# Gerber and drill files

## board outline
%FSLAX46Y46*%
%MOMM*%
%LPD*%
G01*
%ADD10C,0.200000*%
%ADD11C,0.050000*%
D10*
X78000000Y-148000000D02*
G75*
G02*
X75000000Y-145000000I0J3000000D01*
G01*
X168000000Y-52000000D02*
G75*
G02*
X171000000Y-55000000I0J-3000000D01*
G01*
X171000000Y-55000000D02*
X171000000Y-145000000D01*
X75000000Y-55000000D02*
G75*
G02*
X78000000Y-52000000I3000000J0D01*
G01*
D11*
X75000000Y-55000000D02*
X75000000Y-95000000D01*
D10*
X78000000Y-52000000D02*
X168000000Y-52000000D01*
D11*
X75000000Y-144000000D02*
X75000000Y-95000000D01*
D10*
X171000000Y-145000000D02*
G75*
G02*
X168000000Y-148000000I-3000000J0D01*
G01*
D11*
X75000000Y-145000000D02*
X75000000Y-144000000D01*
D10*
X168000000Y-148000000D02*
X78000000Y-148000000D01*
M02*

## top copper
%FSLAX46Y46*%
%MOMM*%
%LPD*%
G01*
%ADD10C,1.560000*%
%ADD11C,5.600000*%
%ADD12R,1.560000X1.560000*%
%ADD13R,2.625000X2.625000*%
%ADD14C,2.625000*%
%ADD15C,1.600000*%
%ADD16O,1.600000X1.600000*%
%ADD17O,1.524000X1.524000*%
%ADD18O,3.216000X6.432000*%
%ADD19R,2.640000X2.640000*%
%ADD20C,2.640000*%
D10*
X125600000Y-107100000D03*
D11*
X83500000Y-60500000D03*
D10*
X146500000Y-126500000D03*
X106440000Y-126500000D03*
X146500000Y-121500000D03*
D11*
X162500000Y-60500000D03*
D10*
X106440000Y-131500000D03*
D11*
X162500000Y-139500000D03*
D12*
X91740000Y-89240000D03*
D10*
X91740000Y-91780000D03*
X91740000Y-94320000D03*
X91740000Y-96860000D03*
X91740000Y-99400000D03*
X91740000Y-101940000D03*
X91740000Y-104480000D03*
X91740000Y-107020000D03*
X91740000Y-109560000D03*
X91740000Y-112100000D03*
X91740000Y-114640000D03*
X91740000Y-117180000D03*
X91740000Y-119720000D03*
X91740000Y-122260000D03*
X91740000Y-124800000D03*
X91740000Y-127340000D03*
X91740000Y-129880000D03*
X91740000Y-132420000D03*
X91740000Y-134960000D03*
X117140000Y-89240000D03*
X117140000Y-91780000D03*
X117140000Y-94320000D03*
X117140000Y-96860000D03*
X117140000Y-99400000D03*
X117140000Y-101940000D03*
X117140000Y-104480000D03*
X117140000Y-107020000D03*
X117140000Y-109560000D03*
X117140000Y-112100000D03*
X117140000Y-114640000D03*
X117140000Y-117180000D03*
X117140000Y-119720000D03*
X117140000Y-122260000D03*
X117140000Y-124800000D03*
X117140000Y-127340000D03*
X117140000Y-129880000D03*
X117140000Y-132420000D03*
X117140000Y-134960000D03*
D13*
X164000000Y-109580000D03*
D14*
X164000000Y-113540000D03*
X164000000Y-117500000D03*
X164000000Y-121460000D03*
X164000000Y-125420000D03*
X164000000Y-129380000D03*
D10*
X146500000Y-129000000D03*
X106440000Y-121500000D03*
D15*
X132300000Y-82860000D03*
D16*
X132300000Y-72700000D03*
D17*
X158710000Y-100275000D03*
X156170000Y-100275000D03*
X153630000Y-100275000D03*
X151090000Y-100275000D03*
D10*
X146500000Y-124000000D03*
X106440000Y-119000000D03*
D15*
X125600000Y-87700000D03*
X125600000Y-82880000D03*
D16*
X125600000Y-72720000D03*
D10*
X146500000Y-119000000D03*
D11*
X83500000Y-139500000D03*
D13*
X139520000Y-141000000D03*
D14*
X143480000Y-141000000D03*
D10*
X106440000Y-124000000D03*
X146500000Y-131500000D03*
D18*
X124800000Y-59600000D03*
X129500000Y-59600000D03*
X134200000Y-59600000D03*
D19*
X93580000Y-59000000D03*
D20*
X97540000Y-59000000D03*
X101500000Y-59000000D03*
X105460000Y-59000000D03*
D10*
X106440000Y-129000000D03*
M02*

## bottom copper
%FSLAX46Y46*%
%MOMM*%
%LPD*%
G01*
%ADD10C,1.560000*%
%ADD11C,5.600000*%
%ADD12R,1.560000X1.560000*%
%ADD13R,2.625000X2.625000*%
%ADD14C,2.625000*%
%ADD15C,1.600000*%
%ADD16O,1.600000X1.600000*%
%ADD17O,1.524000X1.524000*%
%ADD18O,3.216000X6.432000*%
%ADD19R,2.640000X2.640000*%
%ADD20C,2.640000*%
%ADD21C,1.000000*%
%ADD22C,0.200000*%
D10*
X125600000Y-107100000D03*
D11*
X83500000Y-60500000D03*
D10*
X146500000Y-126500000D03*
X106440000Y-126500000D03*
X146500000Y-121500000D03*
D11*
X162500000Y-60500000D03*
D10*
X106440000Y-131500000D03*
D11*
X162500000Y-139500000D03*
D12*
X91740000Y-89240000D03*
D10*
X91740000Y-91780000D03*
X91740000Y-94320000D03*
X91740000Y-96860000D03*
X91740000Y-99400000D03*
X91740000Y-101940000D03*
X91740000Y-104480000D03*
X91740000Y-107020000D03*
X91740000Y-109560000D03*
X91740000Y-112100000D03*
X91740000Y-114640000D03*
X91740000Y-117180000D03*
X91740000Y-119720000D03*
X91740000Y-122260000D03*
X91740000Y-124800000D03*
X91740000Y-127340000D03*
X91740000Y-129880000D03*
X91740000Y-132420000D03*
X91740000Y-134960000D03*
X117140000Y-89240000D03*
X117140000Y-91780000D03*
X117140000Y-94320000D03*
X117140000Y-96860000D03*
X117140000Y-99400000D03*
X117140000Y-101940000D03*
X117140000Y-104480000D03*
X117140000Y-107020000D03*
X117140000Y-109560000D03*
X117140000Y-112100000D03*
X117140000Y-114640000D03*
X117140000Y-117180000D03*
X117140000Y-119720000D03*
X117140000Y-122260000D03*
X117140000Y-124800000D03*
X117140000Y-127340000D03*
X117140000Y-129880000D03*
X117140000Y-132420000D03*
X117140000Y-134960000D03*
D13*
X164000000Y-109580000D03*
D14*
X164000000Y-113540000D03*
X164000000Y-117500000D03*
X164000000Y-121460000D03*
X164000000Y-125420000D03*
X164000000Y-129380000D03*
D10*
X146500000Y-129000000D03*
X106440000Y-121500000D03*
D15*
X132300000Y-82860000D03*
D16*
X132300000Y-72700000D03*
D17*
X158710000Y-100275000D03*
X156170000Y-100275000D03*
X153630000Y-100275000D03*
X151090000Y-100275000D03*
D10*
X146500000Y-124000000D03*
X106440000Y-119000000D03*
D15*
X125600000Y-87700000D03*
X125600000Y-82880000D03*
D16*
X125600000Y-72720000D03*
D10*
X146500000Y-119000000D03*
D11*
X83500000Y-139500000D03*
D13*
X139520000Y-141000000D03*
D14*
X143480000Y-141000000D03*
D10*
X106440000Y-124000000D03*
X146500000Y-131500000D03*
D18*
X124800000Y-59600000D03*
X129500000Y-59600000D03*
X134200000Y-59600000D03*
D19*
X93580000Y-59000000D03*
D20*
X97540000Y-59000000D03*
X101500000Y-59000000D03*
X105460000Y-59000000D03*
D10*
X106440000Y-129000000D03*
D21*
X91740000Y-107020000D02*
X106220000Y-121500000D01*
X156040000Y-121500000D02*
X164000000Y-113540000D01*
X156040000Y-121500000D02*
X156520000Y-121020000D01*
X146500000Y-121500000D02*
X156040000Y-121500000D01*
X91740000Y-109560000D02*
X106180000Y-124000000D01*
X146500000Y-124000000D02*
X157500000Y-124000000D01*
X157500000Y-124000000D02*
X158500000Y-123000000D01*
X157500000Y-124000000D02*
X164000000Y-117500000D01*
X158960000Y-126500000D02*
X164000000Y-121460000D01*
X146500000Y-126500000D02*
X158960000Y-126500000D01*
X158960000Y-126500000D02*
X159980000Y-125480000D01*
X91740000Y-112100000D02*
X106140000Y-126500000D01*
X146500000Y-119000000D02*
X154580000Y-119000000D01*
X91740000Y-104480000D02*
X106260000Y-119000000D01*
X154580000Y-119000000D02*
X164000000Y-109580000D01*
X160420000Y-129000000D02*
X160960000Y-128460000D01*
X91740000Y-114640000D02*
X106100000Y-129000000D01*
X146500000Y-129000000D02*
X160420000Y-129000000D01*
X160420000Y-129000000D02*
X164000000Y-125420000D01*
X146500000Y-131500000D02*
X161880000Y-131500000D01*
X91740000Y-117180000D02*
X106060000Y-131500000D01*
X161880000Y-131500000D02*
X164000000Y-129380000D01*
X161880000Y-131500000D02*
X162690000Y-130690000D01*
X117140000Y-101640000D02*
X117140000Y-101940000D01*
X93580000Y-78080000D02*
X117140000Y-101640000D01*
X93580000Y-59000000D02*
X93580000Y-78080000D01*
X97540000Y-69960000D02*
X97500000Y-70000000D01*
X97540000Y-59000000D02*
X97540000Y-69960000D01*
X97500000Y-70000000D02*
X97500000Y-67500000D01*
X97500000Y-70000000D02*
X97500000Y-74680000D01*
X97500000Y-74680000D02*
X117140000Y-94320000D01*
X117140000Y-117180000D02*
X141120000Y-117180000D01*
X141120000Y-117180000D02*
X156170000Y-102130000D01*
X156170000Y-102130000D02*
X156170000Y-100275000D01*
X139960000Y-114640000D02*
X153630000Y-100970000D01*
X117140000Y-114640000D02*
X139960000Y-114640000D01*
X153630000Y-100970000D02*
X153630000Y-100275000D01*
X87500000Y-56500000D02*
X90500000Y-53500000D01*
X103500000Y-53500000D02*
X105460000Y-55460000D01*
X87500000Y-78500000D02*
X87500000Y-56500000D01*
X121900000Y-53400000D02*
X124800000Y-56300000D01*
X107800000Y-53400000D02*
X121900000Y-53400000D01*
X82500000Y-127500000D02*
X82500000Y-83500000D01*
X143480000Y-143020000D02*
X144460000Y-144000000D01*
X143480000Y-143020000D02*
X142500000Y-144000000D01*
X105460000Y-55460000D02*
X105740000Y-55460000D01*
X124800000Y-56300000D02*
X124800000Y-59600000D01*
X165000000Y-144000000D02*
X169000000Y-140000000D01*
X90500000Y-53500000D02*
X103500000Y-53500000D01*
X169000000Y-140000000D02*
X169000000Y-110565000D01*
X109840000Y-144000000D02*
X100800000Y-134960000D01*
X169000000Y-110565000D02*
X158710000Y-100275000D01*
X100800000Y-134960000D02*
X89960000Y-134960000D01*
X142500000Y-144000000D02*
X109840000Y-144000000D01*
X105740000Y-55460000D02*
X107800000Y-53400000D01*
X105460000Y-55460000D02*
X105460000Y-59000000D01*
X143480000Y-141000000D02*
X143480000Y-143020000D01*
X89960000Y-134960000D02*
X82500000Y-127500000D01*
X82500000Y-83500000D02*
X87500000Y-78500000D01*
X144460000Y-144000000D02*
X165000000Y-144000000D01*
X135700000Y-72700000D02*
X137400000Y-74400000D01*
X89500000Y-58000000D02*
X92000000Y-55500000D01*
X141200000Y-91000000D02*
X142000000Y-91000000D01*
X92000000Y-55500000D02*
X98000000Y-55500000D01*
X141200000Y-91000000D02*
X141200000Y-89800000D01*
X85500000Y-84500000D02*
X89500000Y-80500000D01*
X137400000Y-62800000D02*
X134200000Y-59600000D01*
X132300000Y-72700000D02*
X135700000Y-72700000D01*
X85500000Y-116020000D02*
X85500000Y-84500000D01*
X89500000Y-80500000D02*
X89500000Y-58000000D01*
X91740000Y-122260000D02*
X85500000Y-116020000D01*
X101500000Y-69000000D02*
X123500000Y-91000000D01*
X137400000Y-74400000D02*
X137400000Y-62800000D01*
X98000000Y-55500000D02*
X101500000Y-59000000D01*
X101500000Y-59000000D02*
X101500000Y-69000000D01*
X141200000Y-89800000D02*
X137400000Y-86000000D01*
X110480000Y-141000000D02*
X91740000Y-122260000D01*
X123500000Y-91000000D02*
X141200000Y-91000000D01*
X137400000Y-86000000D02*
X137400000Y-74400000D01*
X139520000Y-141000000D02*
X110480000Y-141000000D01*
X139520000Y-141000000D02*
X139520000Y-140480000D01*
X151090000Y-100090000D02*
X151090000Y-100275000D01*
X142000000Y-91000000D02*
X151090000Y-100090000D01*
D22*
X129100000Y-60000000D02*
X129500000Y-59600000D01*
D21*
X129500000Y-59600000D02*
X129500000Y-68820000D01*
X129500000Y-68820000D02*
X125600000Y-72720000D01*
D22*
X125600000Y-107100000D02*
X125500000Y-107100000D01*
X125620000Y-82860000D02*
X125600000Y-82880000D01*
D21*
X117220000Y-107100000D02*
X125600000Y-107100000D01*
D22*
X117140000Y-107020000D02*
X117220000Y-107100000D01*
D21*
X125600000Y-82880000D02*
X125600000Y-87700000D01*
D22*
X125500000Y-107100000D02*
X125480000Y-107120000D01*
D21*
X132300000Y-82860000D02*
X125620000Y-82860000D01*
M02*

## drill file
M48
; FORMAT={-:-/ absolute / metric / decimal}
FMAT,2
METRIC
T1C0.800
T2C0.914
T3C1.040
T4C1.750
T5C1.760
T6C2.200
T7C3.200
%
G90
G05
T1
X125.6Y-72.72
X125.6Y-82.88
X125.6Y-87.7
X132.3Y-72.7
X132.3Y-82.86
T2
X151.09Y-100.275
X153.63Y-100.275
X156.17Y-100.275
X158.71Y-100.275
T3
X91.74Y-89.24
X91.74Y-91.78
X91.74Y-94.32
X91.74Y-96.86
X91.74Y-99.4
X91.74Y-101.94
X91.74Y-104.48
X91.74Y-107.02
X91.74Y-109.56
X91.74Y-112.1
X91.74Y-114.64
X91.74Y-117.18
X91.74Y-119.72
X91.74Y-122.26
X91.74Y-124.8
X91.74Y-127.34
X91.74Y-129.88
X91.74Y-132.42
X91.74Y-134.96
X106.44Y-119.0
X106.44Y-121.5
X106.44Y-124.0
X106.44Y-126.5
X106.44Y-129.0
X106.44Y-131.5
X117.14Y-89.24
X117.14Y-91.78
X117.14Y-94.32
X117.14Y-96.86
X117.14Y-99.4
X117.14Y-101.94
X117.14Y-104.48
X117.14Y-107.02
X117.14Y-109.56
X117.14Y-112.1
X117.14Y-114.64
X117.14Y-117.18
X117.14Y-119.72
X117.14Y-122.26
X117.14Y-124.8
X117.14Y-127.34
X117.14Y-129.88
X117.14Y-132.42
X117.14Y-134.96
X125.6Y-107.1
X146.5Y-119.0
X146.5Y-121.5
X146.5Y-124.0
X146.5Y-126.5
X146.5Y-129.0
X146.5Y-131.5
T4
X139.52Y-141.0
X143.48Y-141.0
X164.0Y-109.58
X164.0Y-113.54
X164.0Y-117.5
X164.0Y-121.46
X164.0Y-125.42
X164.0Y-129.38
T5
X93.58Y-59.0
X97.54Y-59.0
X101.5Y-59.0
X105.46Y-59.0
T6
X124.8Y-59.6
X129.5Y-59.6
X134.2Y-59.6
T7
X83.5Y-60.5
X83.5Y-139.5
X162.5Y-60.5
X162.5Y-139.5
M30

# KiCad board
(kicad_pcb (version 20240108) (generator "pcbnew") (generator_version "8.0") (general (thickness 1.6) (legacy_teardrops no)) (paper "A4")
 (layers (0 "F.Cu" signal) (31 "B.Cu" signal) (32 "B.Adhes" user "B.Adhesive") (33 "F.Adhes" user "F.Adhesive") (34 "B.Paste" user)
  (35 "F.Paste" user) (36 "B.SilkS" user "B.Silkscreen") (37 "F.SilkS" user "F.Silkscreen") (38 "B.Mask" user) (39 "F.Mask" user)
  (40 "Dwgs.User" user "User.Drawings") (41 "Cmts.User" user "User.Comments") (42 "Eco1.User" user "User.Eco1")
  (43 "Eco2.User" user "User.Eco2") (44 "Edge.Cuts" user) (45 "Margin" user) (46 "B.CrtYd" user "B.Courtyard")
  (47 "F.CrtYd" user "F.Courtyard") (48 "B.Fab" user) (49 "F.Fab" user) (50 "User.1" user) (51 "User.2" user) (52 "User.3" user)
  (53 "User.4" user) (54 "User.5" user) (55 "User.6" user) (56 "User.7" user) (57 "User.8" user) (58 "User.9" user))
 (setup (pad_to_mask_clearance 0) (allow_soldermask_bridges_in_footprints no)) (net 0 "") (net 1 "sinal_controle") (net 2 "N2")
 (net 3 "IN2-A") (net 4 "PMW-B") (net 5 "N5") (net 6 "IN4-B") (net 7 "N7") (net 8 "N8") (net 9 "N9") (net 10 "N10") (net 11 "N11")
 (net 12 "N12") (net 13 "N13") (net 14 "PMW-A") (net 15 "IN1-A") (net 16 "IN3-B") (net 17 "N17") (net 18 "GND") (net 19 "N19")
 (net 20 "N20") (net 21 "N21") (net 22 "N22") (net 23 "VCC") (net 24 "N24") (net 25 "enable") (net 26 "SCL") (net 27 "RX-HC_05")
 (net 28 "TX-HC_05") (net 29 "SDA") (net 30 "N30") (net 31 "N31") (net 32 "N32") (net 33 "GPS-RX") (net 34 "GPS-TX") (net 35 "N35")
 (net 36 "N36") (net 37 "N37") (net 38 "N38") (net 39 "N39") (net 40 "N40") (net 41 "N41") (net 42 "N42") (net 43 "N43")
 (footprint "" (layer "F.Cu") (at 125.6 107.1)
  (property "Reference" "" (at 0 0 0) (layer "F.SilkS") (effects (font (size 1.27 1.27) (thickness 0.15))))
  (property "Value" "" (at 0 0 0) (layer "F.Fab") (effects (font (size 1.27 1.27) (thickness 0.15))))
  (pad "J3-8" thru_hole circle (at 0 0) (size 1.56 1.56) (drill 1.04) (layers "*.Cu" "*.Mask") (remove_unused_layers no)
   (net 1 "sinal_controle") (solder_mask_margin 0.102)))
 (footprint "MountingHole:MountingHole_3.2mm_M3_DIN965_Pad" (layer "F.Cu") (at 83.5 60.5)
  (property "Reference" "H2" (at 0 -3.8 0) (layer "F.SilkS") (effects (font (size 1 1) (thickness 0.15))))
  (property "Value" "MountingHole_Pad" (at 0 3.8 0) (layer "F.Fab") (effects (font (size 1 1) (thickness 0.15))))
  (pad "1" thru_hole circle (at 0 0) (size 5.6 5.6) (drill 3.2) (layers "*.Cu" "*.Mask") (remove_unused_layers no) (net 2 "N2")))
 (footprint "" (layer "F.Cu") (at 146.5 126.5)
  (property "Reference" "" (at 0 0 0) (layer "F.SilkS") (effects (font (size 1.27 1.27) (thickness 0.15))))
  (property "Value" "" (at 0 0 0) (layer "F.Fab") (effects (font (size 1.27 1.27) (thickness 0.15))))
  (pad "J2-10" thru_hole circle (at 0 0) (size 1.56 1.56) (drill 1.04) (layers "*.Cu" "*.Mask") (remove_unused_layers no) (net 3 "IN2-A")
   (solder_mask_margin 0.102)))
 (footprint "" (layer "F.Cu") (at 106.44 126.5)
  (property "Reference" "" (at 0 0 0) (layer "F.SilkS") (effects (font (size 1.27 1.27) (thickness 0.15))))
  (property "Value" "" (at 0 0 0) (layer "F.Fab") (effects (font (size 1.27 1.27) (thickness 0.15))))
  (pad "J2-10" thru_hole circle (at 0 0) (size 1.56 1.56) (drill 1.04) (layers "*.Cu" "*.Mask") (remove_unused_layers no) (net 3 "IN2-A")
   (solder_mask_margin 0.102)))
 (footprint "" (layer "F.Cu") (at 146.5 121.5)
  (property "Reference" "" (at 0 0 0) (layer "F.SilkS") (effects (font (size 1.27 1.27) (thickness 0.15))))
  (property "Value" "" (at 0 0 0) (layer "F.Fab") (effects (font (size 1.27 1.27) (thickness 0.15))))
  (pad "J2-8" thru_hole circle (at 0 0) (size 1.56 1.56) (drill 1.04) (layers "*.Cu" "*.Mask") (remove_unused_layers no) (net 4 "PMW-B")
   (solder_mask_margin 0.102)))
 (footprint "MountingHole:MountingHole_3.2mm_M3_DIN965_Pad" (layer "F.Cu") (at 162.5 60.5)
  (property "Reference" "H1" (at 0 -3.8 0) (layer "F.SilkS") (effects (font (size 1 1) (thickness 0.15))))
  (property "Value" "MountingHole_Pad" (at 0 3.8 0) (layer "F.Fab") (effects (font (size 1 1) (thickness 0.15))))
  (pad "1" thru_hole circle (at 0 0) (size 5.6 5.6) (drill 3.2) (layers "*.Cu" "*.Mask") (remove_unused_layers no) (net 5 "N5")))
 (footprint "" (layer "F.Cu") (at 106.44 131.5)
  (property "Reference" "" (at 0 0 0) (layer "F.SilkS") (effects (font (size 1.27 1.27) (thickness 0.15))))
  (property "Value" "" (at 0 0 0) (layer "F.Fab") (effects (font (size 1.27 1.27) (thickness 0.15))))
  (pad "J2-12" thru_hole circle (at 0 0) (size 1.56 1.56) (drill 1.04) (layers "*.Cu" "*.Mask") (remove_unused_layers no) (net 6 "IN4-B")
   (solder_mask_margin 0.102)))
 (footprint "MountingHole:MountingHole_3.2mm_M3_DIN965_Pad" (layer "F.Cu") (at 162.5 139.5)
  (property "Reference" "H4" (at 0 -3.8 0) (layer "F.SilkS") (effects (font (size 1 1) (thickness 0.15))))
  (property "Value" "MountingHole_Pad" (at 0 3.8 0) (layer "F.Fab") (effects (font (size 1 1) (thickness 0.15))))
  (pad "1" thru_hole circle (at 0 0) (size 5.6 5.6) (drill 3.2) (layers "*.Cu" "*.Mask") (remove_unused_layers no) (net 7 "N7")))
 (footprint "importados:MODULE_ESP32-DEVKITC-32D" (layer "F.Cu") (at 104.44 109)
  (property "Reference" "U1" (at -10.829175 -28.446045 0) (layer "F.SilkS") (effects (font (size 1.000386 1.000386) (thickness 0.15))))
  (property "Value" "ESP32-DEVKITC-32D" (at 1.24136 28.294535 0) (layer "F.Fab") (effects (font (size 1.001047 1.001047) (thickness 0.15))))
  (pad "J2-1" thru_hole rect (at -12.7 -19.76) (size 1.56 1.56) (drill 1.04) (layers "*.Cu" "*.Mask") (remove_unused_layers no) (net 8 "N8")
   (solder_mask_margin 0.102))
  (pad "J2-2" thru_hole circle (at -12.7 -17.22) (size 1.56 1.56) (drill 1.04) (layers "*.Cu" "*.Mask") (remove_unused_layers no)
   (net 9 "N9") (solder_mask_margin 0.102))
  (pad "J2-3" thru_hole circle (at -12.7 -14.68) (size 1.56 1.56) (drill 1.04) (layers "*.Cu" "*.Mask") (remove_unused_layers no)
   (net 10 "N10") (solder_mask_margin 0.102))
  (pad "J2-4" thru_hole circle (at -12.7 -12.14) (size 1.56 1.56) (drill 1.04) (layers "*.Cu" "*.Mask") (remove_unused_layers no)
   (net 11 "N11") (solder_mask_margin 0.102))
  (pad "J2-5" thru_hole circle (at -12.7 -9.6) (size 1.56 1.56) (drill 1.04) (layers "*.Cu" "*.Mask") (remove_unused_layers no)
   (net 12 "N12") (solder_mask_margin 0.102))
  (pad "J2-6" thru_hole circle (at -12.7 -7.06) (size 1.56 1.56) (drill 1.04) (layers "*.Cu" "*.Mask") (remove_unused_layers no)
   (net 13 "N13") (solder_mask_margin 0.102))
  (pad "J2-7" thru_hole circle (at -12.7 -4.52) (size 1.56 1.56) (drill 1.04) (layers "*.Cu" "*.Mask") (remove_unused_layers no)
   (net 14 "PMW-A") (solder_mask_margin 0.102))
  (pad "J2-8" thru_hole circle (at -12.7 -1.98) (size 1.56 1.56) (drill 1.04) (layers "*.Cu" "*.Mask") (remove_unused_layers no)
   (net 4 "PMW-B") (solder_mask_margin 0.102))
  (pad "J2-9" thru_hole circle (at -12.7 0.56) (size 1.56 1.56) (drill 1.04) (layers "*.Cu" "*.Mask") (remove_unused_layers no)
   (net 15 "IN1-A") (solder_mask_margin 0.102))
  (pad "J2-10" thru_hole circle (at -12.7 3.1) (size 1.56 1.56) (drill 1.04) (layers "*.Cu" "*.Mask") (remove_unused_layers no)
   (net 3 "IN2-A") (solder_mask_margin 0.102))
  (pad "J2-11" thru_hole circle (at -12.7 5.64) (size 1.56 1.56) (drill 1.04) (layers "*.Cu" "*.Mask") (remove_unused_layers no)
   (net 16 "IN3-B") (solder_mask_margin 0.102))
  (pad "J2-12" thru_hole circle (at -12.7 8.18) (size 1.56 1.56) (drill 1.04) (layers "*.Cu" "*.Mask") (remove_unused_layers no)
   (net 6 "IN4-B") (solder_mask_margin 0.102))
  (pad "J2-13" thru_hole circle (at -12.7 10.72) (size 1.56 1.56) (drill 1.04) (layers "*.Cu" "*.Mask") (remove_unused_layers no)
   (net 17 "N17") (solder_mask_margin 0.102))
  (pad "J2-14" thru_hole circle (at -12.7 13.26) (size 1.56 1.56) (drill 1.04) (layers "*.Cu" "*.Mask") (remove_unused_layers no)
   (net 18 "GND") (solder_mask_margin 0.102))
  (pad "J2-15" thru_hole circle (at -12.7 15.8) (size 1.56 1.56) (drill 1.04) (layers "*.Cu" "*.Mask") (remove_unused_layers no)
   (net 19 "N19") (solder_mask_margin 0.102))
  (pad "J2-16" thru_hole circle (at -12.7 18.34) (size 1.56 1.56) (drill 1.04) (layers "*.Cu" "*.Mask") (remove_unused_layers no)
   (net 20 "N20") (solder_mask_margin 0.102))
  (pad "J2-17" thru_hole circle (at -12.7 20.88) (size 1.56 1.56) (drill 1.04) (layers "*.Cu" "*.Mask") (remove_unused_layers no)
   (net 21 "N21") (solder_mask_margin 0.102))
  (pad "J2-18" thru_hole circle (at -12.7 23.42) (size 1.56 1.56) (drill 1.04) (layers "*.Cu" "*.Mask") (remove_unused_layers no)
   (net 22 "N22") (solder_mask_margin 0.102))
  (pad "J2-19" thru_hole circle (at -12.7 25.96) (size 1.56 1.56) (drill 1.04) (layers "*.Cu" "*.Mask") (remove_unused_layers no)
   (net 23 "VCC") (solder_mask_margin 0.102))
  (pad "J3-1" thru_hole circle (at 12.7 -19.76) (size 1.56 1.56) (drill 1.04) (layers "*.Cu" "*.Mask") (remove_unused_layers no)
   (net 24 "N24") (solder_mask_margin 0.102))
  (pad "J3-2" thru_hole circle (at 12.7 -17.22) (size 1.56 1.56) (drill 1.04) (layers "*.Cu" "*.Mask") (remove_unused_layers no)
   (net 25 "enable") (solder_mask_margin 0.102))
  (pad "J3-3" thru_hole circle (at 12.7 -14.68) (size 1.56 1.56) (drill 1.04) (layers "*.Cu" "*.Mask") (remove_unused_layers no)
   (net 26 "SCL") (solder_mask_margin 0.102))
  (pad "J3-4" thru_hole circle (at 12.7 -12.14) (size 1.56 1.56) (drill 1.04) (layers "*.Cu" "*.Mask") (remove_unused_layers no)
   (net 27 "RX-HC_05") (solder_mask_margin 0.102))
  (pad "J3-5" thru_hole circle (at 12.7 -9.6) (size 1.56 1.56) (drill 1.04) (layers "*.Cu" "*.Mask") (remove_unused_layers no)
   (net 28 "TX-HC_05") (solder_mask_margin 0.102))
  (pad "J3-6" thru_hole circle (at 12.7 -7.06) (size 1.56 1.56) (drill 1.04) (layers "*.Cu" "*.Mask") (remove_unused_layers no)
   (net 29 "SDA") (solder_mask_margin 0.102))
  (pad "J3-7" thru_hole circle (at 12.7 -4.52) (size 1.56 1.56) (drill 1.04) (layers "*.Cu" "*.Mask") (remove_unused_layers no)
   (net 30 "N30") (solder_mask_margin 0.102))
  (pad "J3-8" thru_hole circle (at 12.7 -1.98) (size 1.56 1.56) (drill 1.04) (layers "*.Cu" "*.Mask") (remove_unused_layers no)
   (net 1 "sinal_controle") (solder_mask_margin 0.102))
  (pad "J3-9" thru_hole circle (at 12.7 0.56) (size 1.56 1.56) (drill 1.04) (layers "*.Cu" "*.Mask") (remove_unused_layers no)
   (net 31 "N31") (solder_mask_margin 0.102))
  (pad "J3-10" thru_hole circle (at 12.7 3.1) (size 1.56 1.56) (drill 1.04) (layers "*.Cu" "*.Mask") (remove_unused_layers no)
   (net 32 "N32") (solder_mask_margin 0.102))
  (pad "J3-11" thru_hole circle (at 12.7 5.64) (size 1.56 1.56) (drill 1.04) (layers "*.Cu" "*.Mask") (remove_unused_layers no)
   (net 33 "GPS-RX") (solder_mask_margin 0.102))
  (pad "J3-12" thru_hole circle (at 12.7 8.18) (size 1.56 1.56) (drill 1.04) (layers "*.Cu" "*.Mask") (remove_unused_layers no)
   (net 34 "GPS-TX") (solder_mask_margin 0.102))
  (pad "J3-13" thru_hole circle (at 12.7 10.72) (size 1.56 1.56) (drill 1.04) (layers "*.Cu" "*.Mask") (remove_unused_layers no)
   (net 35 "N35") (solder_mask_margin 0.102))
  (pad "J3-14" thru_hole circle (at 12.7 13.26) (size 1.56 1.56) (drill 1.04) (layers "*.Cu" "*.Mask") (remove_unused_layers no)
   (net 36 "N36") (solder_mask_margin 0.102))
  (pad "J3-15" thru_hole circle (at 12.7 15.8) (size 1.56 1.56) (drill 1.04) (layers "*.Cu" "*.Mask") (remove_unused_layers no)
   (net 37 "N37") (solder_mask_margin 0.102))
  (pad "J3-16" thru_hole circle (at 12.7 18.34) (size 1.56 1.56) (drill 1.04) (layers "*.Cu" "*.Mask") (remove_unused_layers no)
   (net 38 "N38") (solder_mask_margin 0.102))
  (pad "J3-17" thru_hole circle (at 12.7 20.88) (size 1.56 1.56) (drill 1.04) (layers "*.Cu" "*.Mask") (remove_unused_layers no)
   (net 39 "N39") (solder_mask_margin 0.102))
  (pad "J3-18" thru_hole circle (at 12.7 23.42) (size 1.56 1.56) (drill 1.04) (layers "*.Cu" "*.Mask") (remove_unused_layers no)
   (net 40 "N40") (solder_mask_margin 0.102))
  (pad "J3-19" thru_hole circle (at 12.7 25.96) (size 1.56 1.56) (drill 1.04) (layers "*.Cu" "*.Mask") (remove_unused_layers no)
   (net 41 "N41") (solder_mask_margin 0.102)))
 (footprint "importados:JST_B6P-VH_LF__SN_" (layer "F.Cu") (at 164 119.48 -90)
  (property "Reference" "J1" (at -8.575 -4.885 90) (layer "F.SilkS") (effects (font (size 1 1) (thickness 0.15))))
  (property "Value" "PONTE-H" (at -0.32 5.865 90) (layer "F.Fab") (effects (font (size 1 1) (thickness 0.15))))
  (pad "1" thru_hole rect (at -9.9 0 270) (size 2.625 2.625) (drill 1.75) (layers "*.Cu" "*.Mask") (remove_unused_layers no)
   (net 14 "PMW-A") (solder_mask_margin 0.102))
  (pad "2" thru_hole circle (at -5.94 0 270) (size 2.625 2.625) (drill 1.75) (layers "*.Cu" "*.Mask") (remove_unused_layers no)
   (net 4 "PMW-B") (solder_mask_margin 0.102))
  (pad "3" thru_hole circle (at -1.98 0 270) (size 2.625 2.625) (drill 1.75) (layers "*.Cu" "*.Mask") (remove_unused_layers no)
   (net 15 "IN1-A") (solder_mask_margin 0.102))
  (pad "4" thru_hole circle (at 1.98 0 270) (size 2.625 2.625) (drill 1.75) (layers "*.Cu" "*.Mask") (remove_unused_layers no)
   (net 3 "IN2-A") (solder_mask_margin 0.102))
  (pad "5" thru_hole circle (at 5.94 0 270) (size 2.625 2.625) (drill 1.75) (layers "*.Cu" "*.Mask") (remove_unused_layers no)
   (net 16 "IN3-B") (solder_mask_margin 0.102))
  (pad "6" thru_hole circle (at 9.9 0 270) (size 2.625 2.625) (drill 1.75) (layers "*.Cu" "*.Mask") (remove_unused_layers no)
   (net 6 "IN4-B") (solder_mask_margin 0.102)))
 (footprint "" (layer "F.Cu") (at 146.5 129)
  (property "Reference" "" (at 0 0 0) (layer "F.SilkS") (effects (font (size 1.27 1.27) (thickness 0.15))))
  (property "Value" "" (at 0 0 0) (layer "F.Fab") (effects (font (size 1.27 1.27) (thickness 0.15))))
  (pad "J2-11" thru_hole circle (at 0 0) (size 1.56 1.56) (drill 1.04) (layers "*.Cu" "*.Mask") (remove_unused_layers no) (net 16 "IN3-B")
   (solder_mask_margin 0.102)))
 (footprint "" (layer "F.Cu") (at 106.44 121.5)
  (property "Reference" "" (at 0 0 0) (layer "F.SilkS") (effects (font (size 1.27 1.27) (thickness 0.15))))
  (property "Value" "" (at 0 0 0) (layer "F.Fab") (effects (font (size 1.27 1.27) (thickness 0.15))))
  (pad "J2-8" thru_hole circle (at 0 0) (size 1.56 1.56) (drill 1.04) (layers "*.Cu" "*.Mask") (remove_unused_layers no) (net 4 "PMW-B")
   (solder_mask_margin 0.102)))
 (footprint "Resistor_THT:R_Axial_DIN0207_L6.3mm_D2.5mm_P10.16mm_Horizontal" (layer "F.Cu") (at 132.3 82.86 90)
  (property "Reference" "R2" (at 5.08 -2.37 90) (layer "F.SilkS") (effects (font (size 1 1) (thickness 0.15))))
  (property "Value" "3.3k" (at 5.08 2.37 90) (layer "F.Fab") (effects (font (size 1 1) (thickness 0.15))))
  (pad "1" thru_hole circle (at 0 0 90) (size 1.6 1.6) (drill 0.8) (layers "*.Cu" "*.Mask") (remove_unused_layers no)
   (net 1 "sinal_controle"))
  (pad "2" thru_hole oval (at 10.16 0 90) (size 1.6 1.6) (drill 0.8) (layers "*.Cu" "*.Mask") (remove_unused_layers no) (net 18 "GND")))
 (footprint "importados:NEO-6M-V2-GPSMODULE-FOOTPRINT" (layer "F.Cu") (at 154.9 84.4 180)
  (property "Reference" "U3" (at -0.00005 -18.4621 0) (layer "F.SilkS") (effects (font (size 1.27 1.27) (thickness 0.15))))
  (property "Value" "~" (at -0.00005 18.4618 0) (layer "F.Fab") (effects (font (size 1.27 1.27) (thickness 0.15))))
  (pad "1" thru_hole oval (at -3.81 -15.875 180) (size 1.524 1.524) (drill 0.9144) (layers "*.Cu" "*.Mask") (remove_unused_layers no)
   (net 23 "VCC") (solder_mask_margin 0.254) (thermal_bridge_angle 0))
  (pad "2" thru_hole oval (at -1.27 -15.875 180) (size 1.524 1.524) (drill 0.9144) (layers "*.Cu" "*.Mask") (remove_unused_layers no)
   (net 34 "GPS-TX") (solder_mask_margin 0.254) (thermal_bridge_angle 0))
  (pad "3" thru_hole oval (at 1.27 -15.875 180) (size 1.524 1.524) (drill 0.9144) (layers "*.Cu" "*.Mask") (remove_unused_layers no)
   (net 33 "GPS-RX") (solder_mask_margin 0.254) (thermal_bridge_angle 0))
  (pad "4" thru_hole oval (at 3.81 -15.875 180) (size 1.524 1.524) (drill 0.9144) (layers "*.Cu" "*.Mask") (remove_unused_layers no)
   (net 18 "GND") (solder_mask_margin 0.254) (thermal_bridge_angle 0))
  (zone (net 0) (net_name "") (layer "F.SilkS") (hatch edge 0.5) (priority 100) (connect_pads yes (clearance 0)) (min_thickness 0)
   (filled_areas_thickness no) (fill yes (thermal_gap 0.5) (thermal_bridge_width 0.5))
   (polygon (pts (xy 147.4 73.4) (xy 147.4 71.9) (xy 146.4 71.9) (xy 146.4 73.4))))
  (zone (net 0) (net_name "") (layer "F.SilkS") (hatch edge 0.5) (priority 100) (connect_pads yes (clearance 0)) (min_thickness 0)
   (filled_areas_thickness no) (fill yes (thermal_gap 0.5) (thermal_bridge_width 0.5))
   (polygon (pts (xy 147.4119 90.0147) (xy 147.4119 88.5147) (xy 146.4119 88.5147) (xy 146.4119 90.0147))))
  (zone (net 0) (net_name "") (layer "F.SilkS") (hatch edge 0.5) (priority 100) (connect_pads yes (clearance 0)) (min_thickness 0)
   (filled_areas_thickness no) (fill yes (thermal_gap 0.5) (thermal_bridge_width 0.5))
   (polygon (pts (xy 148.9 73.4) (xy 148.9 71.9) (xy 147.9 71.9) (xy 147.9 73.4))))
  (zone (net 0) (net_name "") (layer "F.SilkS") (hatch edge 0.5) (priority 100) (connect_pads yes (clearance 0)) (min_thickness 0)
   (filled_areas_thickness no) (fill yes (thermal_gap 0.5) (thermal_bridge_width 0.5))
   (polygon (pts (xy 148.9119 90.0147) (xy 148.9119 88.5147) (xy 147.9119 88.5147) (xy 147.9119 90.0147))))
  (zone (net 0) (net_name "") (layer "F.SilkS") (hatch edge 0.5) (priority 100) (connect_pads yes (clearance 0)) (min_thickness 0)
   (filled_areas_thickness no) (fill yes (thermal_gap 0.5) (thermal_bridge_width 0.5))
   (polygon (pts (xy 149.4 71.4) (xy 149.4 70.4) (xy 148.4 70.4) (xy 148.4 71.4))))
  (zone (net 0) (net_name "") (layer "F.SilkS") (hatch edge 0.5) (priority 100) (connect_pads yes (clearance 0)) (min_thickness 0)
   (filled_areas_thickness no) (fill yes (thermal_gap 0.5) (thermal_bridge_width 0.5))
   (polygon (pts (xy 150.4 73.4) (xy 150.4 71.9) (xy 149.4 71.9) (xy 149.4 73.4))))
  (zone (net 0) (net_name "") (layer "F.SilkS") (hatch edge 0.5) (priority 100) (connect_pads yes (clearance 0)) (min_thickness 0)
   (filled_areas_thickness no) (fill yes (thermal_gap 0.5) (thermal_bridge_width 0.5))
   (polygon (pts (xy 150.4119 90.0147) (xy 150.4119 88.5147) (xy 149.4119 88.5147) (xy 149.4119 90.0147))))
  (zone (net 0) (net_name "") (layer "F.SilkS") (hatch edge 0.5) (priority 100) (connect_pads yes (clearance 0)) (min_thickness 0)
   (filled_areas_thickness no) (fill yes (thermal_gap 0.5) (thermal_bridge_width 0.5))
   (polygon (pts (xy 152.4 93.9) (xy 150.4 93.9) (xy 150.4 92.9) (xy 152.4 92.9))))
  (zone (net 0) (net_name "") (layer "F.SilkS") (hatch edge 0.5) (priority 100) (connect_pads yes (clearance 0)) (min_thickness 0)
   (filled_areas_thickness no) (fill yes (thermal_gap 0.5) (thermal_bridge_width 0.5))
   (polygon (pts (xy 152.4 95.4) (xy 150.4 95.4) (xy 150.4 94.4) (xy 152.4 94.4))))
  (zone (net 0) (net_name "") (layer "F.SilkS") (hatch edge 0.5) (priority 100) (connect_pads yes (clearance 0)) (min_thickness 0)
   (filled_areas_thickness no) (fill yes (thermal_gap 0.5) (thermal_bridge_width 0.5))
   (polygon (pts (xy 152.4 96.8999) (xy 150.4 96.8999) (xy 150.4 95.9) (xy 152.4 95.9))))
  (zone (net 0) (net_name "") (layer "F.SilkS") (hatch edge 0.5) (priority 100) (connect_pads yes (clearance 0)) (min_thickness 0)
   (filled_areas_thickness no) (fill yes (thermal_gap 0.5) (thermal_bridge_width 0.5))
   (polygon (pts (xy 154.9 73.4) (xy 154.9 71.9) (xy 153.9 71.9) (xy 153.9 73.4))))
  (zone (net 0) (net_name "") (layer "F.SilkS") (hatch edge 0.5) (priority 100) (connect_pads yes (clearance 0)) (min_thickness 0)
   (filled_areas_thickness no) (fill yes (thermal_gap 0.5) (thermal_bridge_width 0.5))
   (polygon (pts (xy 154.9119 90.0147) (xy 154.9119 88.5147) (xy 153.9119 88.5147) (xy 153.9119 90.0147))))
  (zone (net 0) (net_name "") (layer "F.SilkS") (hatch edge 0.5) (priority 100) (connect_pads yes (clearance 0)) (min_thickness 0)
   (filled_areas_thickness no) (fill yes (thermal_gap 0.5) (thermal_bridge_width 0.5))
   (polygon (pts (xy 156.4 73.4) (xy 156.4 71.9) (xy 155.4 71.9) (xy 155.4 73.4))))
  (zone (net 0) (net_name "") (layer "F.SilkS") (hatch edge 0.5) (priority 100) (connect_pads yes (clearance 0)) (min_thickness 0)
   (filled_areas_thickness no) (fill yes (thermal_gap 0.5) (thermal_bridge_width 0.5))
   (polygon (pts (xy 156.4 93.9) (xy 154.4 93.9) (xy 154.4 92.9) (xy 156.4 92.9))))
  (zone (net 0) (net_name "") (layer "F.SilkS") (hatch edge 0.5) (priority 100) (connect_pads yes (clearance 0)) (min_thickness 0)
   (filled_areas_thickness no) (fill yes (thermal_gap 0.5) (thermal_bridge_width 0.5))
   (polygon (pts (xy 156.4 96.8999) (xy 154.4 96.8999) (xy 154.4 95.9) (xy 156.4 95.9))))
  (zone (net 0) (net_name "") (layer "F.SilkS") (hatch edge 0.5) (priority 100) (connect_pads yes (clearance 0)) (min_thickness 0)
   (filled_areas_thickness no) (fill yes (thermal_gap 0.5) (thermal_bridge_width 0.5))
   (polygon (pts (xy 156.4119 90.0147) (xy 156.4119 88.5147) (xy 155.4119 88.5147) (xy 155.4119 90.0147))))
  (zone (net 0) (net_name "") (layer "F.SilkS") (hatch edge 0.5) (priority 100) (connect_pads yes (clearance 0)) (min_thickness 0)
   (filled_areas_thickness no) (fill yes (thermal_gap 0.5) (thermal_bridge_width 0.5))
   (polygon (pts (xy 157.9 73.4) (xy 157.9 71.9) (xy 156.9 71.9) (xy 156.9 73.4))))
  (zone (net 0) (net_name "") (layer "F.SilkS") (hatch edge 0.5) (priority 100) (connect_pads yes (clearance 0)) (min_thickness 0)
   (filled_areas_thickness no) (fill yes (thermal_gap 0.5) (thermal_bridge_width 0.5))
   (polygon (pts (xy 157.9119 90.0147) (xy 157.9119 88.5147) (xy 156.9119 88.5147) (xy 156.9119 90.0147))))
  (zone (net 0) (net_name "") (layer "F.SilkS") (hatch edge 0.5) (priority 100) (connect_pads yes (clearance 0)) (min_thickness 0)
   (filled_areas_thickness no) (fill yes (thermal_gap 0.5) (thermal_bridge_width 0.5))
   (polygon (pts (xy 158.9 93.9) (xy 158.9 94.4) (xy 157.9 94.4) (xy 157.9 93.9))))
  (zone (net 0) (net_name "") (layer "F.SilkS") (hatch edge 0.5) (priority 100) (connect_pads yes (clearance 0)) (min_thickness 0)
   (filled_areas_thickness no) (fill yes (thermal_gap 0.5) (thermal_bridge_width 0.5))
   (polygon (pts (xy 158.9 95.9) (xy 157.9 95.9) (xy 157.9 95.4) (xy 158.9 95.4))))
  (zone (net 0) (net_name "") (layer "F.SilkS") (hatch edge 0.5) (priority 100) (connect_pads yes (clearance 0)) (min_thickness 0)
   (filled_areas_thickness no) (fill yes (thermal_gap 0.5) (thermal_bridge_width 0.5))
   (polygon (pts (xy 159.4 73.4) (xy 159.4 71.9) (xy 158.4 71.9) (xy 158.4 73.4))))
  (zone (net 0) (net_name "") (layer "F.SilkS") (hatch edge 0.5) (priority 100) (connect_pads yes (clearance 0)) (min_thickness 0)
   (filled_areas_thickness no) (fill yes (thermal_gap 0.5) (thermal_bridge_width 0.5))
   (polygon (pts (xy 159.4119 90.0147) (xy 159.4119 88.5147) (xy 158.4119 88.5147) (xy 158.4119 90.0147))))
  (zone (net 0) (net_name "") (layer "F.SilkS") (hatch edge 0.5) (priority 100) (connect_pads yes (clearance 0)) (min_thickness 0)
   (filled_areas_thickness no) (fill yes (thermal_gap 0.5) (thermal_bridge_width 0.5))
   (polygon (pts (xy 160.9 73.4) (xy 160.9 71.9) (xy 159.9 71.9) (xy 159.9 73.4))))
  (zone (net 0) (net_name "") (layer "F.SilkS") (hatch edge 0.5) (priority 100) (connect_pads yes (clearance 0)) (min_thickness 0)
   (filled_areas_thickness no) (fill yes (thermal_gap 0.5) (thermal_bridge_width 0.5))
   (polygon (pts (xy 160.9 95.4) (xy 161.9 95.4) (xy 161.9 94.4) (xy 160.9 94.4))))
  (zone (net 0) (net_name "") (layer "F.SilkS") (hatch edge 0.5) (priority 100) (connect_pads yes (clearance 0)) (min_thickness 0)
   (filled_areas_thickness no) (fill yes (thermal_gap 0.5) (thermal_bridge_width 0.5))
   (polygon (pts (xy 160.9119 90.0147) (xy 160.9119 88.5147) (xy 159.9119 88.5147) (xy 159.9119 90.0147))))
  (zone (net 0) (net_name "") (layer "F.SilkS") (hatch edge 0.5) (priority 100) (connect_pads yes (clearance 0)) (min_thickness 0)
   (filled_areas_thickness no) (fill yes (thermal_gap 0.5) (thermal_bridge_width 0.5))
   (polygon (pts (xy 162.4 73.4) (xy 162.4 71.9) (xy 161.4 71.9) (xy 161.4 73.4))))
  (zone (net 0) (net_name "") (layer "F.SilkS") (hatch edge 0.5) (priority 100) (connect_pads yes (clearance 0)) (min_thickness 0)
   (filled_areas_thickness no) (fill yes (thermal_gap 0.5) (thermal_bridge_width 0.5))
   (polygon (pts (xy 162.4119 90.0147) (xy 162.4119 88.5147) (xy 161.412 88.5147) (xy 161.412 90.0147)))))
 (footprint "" (layer "F.Cu") (at 146.5 124)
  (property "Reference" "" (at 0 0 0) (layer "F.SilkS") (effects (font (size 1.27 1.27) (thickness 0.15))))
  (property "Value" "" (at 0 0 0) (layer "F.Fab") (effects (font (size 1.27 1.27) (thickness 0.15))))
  (pad "J2-9" thru_hole circle (at 0 0) (size 1.56 1.56) (drill 1.04) (layers "*.Cu" "*.Mask") (remove_unused_layers no) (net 15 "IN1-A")
   (solder_mask_margin 0.102)))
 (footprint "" (layer "F.Cu") (at 106.44 119)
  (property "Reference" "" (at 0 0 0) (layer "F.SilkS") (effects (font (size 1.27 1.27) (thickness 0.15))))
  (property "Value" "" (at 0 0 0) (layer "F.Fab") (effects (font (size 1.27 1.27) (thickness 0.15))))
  (pad "J2-7" thru_hole circle (at 0 0) (size 1.56 1.56) (drill 1.04) (layers "*.Cu" "*.Mask") (remove_unused_layers no) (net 14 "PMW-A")
   (solder_mask_margin 0.102)))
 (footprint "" (layer "F.Cu") (at 125.6 87.7)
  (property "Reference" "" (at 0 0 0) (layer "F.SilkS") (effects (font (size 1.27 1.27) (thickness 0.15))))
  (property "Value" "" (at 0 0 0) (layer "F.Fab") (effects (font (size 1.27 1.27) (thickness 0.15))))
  (pad "1" thru_hole circle (at 0 0 90) (size 1.6 1.6) (drill 0.8) (layers "*.Cu" "*.Mask") (remove_unused_layers no)
   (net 1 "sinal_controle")))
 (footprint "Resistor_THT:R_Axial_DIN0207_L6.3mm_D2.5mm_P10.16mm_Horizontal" (layer "F.Cu") (at 125.6 82.88 90)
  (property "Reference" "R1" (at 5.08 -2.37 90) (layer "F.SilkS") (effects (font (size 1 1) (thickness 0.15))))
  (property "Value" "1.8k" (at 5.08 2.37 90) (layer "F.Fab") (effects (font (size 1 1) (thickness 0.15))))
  (pad "1" thru_hole circle (at 0 0 90) (size 1.6 1.6) (drill 0.8) (layers "*.Cu" "*.Mask") (remove_unused_layers no)
   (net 1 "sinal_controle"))
  (pad "2" thru_hole oval (at 10.16 0 90) (size 1.6 1.6) (drill 0.8) (layers "*.Cu" "*.Mask") (remove_unused_layers no) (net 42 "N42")))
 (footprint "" (layer "F.Cu") (at 146.5 119)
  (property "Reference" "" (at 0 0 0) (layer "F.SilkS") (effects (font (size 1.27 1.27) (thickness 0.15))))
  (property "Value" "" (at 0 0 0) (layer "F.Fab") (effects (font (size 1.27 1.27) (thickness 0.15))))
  (pad "J2-7" thru_hole circle (at 0 0) (size 1.56 1.56) (drill 1.04) (layers "*.Cu" "*.Mask") (remove_unused_layers no) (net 14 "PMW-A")
   (solder_mask_margin 0.102)))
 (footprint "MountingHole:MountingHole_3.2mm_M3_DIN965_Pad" (layer "F.Cu") (at 83.5 139.5)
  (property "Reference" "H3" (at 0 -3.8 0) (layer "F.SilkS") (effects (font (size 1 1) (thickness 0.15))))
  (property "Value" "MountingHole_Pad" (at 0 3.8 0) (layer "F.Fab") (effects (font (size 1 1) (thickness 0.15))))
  (pad "1" thru_hole circle (at 0 0) (size 5.6 5.6) (drill 3.2) (layers "*.Cu" "*.Mask") (remove_unused_layers no) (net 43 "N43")))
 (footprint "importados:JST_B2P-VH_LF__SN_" (layer "F.Cu") (at 141.5 141)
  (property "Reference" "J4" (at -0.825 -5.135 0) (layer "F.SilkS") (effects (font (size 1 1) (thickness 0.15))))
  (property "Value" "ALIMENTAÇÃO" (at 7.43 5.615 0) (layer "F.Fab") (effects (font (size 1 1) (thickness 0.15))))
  (pad "1" thru_hole rect (at -1.98 0) (size 2.625 2.625) (drill 1.75) (layers "*.Cu" "*.Mask") (remove_unused_layers no) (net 18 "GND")
   (solder_mask_margin 0.102))
  (pad "2" thru_hole circle (at 1.98 0) (size 2.625 2.625) (drill 1.75) (layers "*.Cu" "*.Mask") (remove_unused_layers no) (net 23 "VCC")
   (solder_mask_margin 0.102)))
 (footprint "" (layer "F.Cu") (at 106.44 124)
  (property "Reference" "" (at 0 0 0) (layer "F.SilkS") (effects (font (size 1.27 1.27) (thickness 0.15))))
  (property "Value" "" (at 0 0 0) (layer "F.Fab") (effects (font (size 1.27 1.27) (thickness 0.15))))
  (pad "J2-9" thru_hole circle (at 0 0) (size 1.56 1.56) (drill 1.04) (layers "*.Cu" "*.Mask") (remove_unused_layers no) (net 15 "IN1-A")
   (solder_mask_margin 0.102)))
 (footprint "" (layer "F.Cu") (at 146.5 131.5)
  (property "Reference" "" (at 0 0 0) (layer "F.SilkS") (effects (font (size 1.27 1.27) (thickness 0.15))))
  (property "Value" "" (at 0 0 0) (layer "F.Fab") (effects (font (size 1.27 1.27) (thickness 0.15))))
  (pad "J2-12" thru_hole circle (at 0 0) (size 1.56 1.56) (drill 1.04) (layers "*.Cu" "*.Mask") (remove_unused_layers no) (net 6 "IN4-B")
   (solder_mask_margin 0.102)))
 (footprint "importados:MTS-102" (layer "F.Cu") (at 129.5 59.6 90)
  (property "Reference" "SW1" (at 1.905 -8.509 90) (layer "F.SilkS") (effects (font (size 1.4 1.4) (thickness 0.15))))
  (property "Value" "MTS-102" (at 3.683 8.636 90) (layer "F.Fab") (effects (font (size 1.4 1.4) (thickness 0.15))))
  (pad "1" thru_hole oval (at 0 -4.7 90) (size 6.432 3.216) (drill 2.2) (layers "*.Cu" "*.Mask") (remove_unused_layers no) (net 23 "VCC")
   (solder_mask_margin 0.102))
  (pad "2" thru_hole oval (at 0 0 90) (size 6.432 3.216) (drill 2.2) (layers "*.Cu" "*.Mask") (remove_unused_layers no) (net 42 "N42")
   (solder_mask_margin 0.102))
  (pad "3" thru_hole oval (at 0 4.7 90) (size 6.432 3.216) (drill 2.2) (layers "*.Cu" "*.Mask") (remove_unused_layers no) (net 18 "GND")
   (solder_mask_margin 0.102)))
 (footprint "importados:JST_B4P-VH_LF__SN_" (layer "F.Cu") (at 99.52 59)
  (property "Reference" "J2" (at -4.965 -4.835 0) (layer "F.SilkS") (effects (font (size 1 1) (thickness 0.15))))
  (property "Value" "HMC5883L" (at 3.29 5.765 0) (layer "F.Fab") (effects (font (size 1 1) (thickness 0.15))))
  (pad "1" thru_hole rect (at -5.94 0) (size 2.64 2.64) (drill 1.76) (layers "*.Cu" "*.Mask") (remove_unused_layers no) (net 29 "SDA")
   (solder_mask_margin 0.102))
  (pad "2" thru_hole circle (at -1.98 0) (size 2.64 2.64) (drill 1.76) (layers "*.Cu" "*.Mask") (remove_unused_layers no) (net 26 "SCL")
   (solder_mask_margin 0.102))
  (pad "3" thru_hole circle (at 1.98 0) (size 2.64 2.64) (drill 1.76) (layers "*.Cu" "*.Mask") (remove_unused_layers no) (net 18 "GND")
   (solder_mask_margin 0.102))
  (pad "4" thru_hole circle (at 5.94 0) (size 2.64 2.64) (drill 1.76) (layers "*.Cu" "*.Mask") (remove_unused_layers no) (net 23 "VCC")
   (solder_mask_margin 0.102)))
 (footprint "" (layer "F.Cu") (at 106.44 129)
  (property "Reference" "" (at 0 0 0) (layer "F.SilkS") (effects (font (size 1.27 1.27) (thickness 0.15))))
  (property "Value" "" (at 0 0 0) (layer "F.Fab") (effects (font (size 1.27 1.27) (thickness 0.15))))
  (pad "J2-11" thru_hole circle (at 0 0) (size 1.56 1.56) (drill 1.04) (layers "*.Cu" "*.Mask") (remove_unused_layers no) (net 16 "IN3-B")
   (solder_mask_margin 0.102)))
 (gr_arc (start 78 148) (mid 75.87868 147.12132) (end 75 145) (stroke (width 0.2) (type default)) (layer "Edge.Cuts"))
 (gr_arc (start 168 52) (mid 170.12132 52.87868) (end 171 55) (stroke (width 0.2) (type default)) (layer "Edge.Cuts"))
 (gr_line (start 171 55) (end 171 145) (stroke (width 0.2) (type default)) (layer "Edge.Cuts"))
 (gr_arc (start 75 55) (mid 75.87868 52.87868) (end 78 52) (stroke (width 0.2) (type default)) (layer "Edge.Cuts"))
 (gr_line (start 75 55) (end 75 95) (stroke (width 0.05) (type default)) (layer "Edge.Cuts"))
 (gr_line (start 78 52) (end 168 52) (stroke (width 0.2) (type default)) (layer "Edge.Cuts"))
 (gr_line (start 75 144) (end 75 95) (stroke (width 0.05) (type default)) (layer "Edge.Cuts"))
 (gr_arc (start 171 145) (mid 170.12132 147.12132) (end 168 148) (stroke (width 0.2) (type default)) (layer "Edge.Cuts"))
 (gr_line (start 75 145) (end 75 144) (stroke (width 0.05) (type default)) (layer "Edge.Cuts"))
 (gr_line (start 168 148) (end 78 148) (stroke (width 0.2) (type default)) (layer "Edge.Cuts"))
 (segment (start 91.74 107.02) (end 106.22 121.5) (width 1) (layer "B.Cu") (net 4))
 (segment (start 156.04 121.5) (end 164 113.54) (width 1) (layer "B.Cu") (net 4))
 (segment (start 156.04 121.5) (end 156.52 121.02) (width 1) (layer "B.Cu") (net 4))
 (segment (start 146.5 121.5) (end 156.04 121.5) (width 1) (layer "B.Cu") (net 4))
 (segment (start 91.74 109.56) (end 106.18 124) (width 1) (layer "B.Cu") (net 15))
 (segment (start 146.5 124) (end 157.5 124) (width 1) (layer "B.Cu") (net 15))
 (segment (start 157.5 124) (end 158.5 123) (width 1) (layer "B.Cu") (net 15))
 (segment (start 157.5 124) (end 164 117.5) (width 1) (layer "B.Cu") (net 15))
 (segment (start 158.96 126.5) (end 164 121.46) (width 1) (layer "B.Cu") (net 3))
 (segment (start 146.5 126.5) (end 158.96 126.5) (width 1) (layer "B.Cu") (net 3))
 (segment (start 158.96 126.5) (end 159.98 125.48) (width 1) (layer "B.Cu") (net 3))
 (segment (start 91.74 112.1) (end 106.14 126.5) (width 1) (layer "B.Cu") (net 3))
 (segment (start 146.5 119) (end 154.58 119) (width 1) (layer "B.Cu") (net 14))
 (segment (start 91.74 104.48) (end 106.26 119) (width 1) (layer "B.Cu") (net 14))
 (segment (start 154.58 119) (end 164 109.58) (width 1) (layer "B.Cu") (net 14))
 (segment (start 160.42 129) (end 160.96 128.46) (width 1) (layer "B.Cu") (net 16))
 (segment (start 91.74 114.64) (end 106.1 129) (width 1) (layer "B.Cu") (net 16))
 (segment (start 146.5 129) (end 160.42 129) (width 1) (layer "B.Cu") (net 16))
 (segment (start 160.42 129) (end 164 125.42) (width 1) (layer "B.Cu") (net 16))
 (segment (start 146.5 131.5) (end 161.88 131.5) (width 1) (layer "B.Cu") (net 6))
 (segment (start 91.74 117.18) (end 106.06 131.5) (width 1) (layer "B.Cu") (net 6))
 (segment (start 161.88 131.5) (end 164 129.38) (width 1) (layer "B.Cu") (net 6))
 (segment (start 161.88 131.5) (end 162.69 130.69) (width 1) (layer "B.Cu") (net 6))
 (segment (start 117.14 101.64) (end 117.14 101.94) (width 1) (layer "B.Cu") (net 29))
 (segment (start 93.58 78.08) (end 117.14 101.64) (width 1) (layer "B.Cu") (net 29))
 (segment (start 93.58 59) (end 93.58 78.08) (width 1) (layer "B.Cu") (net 29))
 (segment (start 97.54 69.96) (end 97.5 70) (width 1) (layer "B.Cu") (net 26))
 (segment (start 97.54 59) (end 97.54 69.96) (width 1) (layer "B.Cu") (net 26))
 (segment (start 97.5 70) (end 97.5 67.5) (width 1) (layer "B.Cu") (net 26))
 (segment (start 97.5 70) (end 97.5 74.68) (width 1) (layer "B.Cu") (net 26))
 (segment (start 97.5 74.68) (end 117.14 94.32) (width 1) (layer "B.Cu") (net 26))
 (segment (start 117.14 117.18) (end 141.12 117.18) (width 1) (layer "B.Cu") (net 34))
 (segment (start 141.12 117.18) (end 156.17 102.13) (width 1) (layer "B.Cu") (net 34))
 (segment (start 156.17 102.13) (end 156.17 100.275) (width 1) (layer "B.Cu") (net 34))
 (segment (start 139.96 114.64) (end 153.63 100.97) (width 1) (layer "B.Cu") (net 33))
 (segment (start 117.14 114.64) (end 139.96 114.64) (width 1) (layer "B.Cu") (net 33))
 (segment (start 153.63 100.97) (end 153.63 100.275) (width 1) (layer "B.Cu") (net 33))
 (segment (start 87.5 56.5) (end 90.5 53.5) (width 1) (layer "B.Cu") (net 23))
 (segment (start 103.5 53.5) (end 105.46 55.46) (width 1) (layer "B.Cu") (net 23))
 (segment (start 87.5 78.5) (end 87.5 56.5) (width 1) (layer "B.Cu") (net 23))
 (segment (start 121.9 53.4) (end 124.8 56.3) (width 1) (layer "B.Cu") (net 23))
 (segment (start 107.8 53.4) (end 121.9 53.4) (width 1) (layer "B.Cu") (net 23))
 (segment (start 82.5 127.5) (end 82.5 83.5) (width 1) (layer "B.Cu") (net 23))
 (segment (start 143.48 143.02) (end 144.46 144) (width 1) (layer "B.Cu") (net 23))
 (segment (start 143.48 143.02) (end 142.5 144) (width 1) (layer "B.Cu") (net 23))
 (segment (start 105.46 55.46) (end 105.74 55.46) (width 1) (layer "B.Cu") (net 23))
 (segment (start 124.8 56.3) (end 124.8 59.6) (width 1) (layer "B.Cu") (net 23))
 (segment (start 165 144) (end 169 140) (width 1) (layer "B.Cu") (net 23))
 (segment (start 90.5 53.5) (end 103.5 53.5) (width 1) (layer "B.Cu") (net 23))
 (segment (start 169 140) (end 169 110.565) (width 1) (layer "B.Cu") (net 23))
 (segment (start 109.84 144) (end 100.8 134.96) (width 1) (layer "B.Cu") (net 23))
 (segment (start 169 110.565) (end 158.71 100.275) (width 1) (layer "B.Cu") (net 23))
 (segment (start 100.8 134.96) (end 89.96 134.96) (width 1) (layer "B.Cu") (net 23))
 (segment (start 142.5 144) (end 109.84 144) (width 1) (layer "B.Cu") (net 23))
 (segment (start 105.74 55.46) (end 107.8 53.4) (width 1) (layer "B.Cu") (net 23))
 (segment (start 105.46 55.46) (end 105.46 59) (width 1) (layer "B.Cu") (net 23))
 (segment (start 143.48 141) (end 143.48 143.02) (width 1) (layer "B.Cu") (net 23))
 (segment (start 89.96 134.96) (end 82.5 127.5) (width 1) (layer "B.Cu") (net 23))
 (segment (start 82.5 83.5) (end 87.5 78.5) (width 1) (layer "B.Cu") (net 23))
 (segment (start 144.46 144) (end 165 144) (width 1) (layer "B.Cu") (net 23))
 (segment (start 135.7 72.7) (end 137.4 74.4) (width 1) (layer "B.Cu") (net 18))
 (segment (start 89.5 58) (end 92 55.5) (width 1) (layer "B.Cu") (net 18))
 (segment (start 141.2 91) (end 142 91) (width 1) (layer "B.Cu") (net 18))
 (segment (start 92 55.5) (end 98 55.5) (width 1) (layer "B.Cu") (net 18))
 (segment (start 141.2 91) (end 141.2 89.8) (width 1) (layer "B.Cu") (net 18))
 (segment (start 85.5 84.5) (end 89.5 80.5) (width 1) (layer "B.Cu") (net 18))
 (segment (start 137.4 62.8) (end 134.2 59.6) (width 1) (layer "B.Cu") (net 18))
 (segment (start 132.3 72.7) (end 135.7 72.7) (width 1) (layer "B.Cu") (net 18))
 (segment (start 85.5 116.02) (end 85.5 84.5) (width 1) (layer "B.Cu") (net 18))
 (segment (start 89.5 80.5) (end 89.5 58) (width 1) (layer "B.Cu") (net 18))
 (segment (start 91.74 122.26) (end 85.5 116.02) (width 1) (layer "B.Cu") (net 18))
 (segment (start 101.5 69) (end 123.5 91) (width 1) (layer "B.Cu") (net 18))
 (segment (start 137.4 74.4) (end 137.4 62.8) (width 1) (layer "B.Cu") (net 18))
 (segment (start 98 55.5) (end 101.5 59) (width 1) (layer "B.Cu") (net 18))
 (segment (start 101.5 59) (end 101.5 69) (width 1) (layer "B.Cu") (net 18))
 (segment (start 141.2 89.8) (end 137.4 86) (width 1) (layer "B.Cu") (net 18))
 (segment (start 110.48 141) (end 91.74 122.26) (width 1) (layer "B.Cu") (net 18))
 (segment (start 123.5 91) (end 141.2 91) (width 1) (layer "B.Cu") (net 18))
 (segment (start 137.4 86) (end 137.4 74.4) (width 1) (layer "B.Cu") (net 18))
 (segment (start 139.52 141) (end 110.48 141) (width 1) (layer "B.Cu") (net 18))
 (segment (start 139.52 141) (end 139.52 140.48) (width 1) (layer "B.Cu") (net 18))
 (segment (start 151.09 100.09) (end 151.09 100.275) (width 1) (layer "B.Cu") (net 18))
 (segment (start 142 91) (end 151.09 100.09) (width 1) (layer "B.Cu") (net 18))
 (segment (start 129.1 60) (end 129.5 59.6) (width 0.2) (layer "B.Cu") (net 42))
 (segment (start 129.5 59.6) (end 129.5 68.82) (width 1) (layer "B.Cu") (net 42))
 (segment (start 129.5 68.82) (end 125.6 72.72) (width 1) (layer "B.Cu") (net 42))
 (segment (start 125.6 107.1) (end 125.5 107.1) (width 0.2) (layer "B.Cu") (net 1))
 (segment (start 125.62 82.86) (end 125.6 82.88) (width 0.2) (layer "B.Cu") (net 1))
 (segment (start 117.22 107.1) (end 125.6 107.1) (width 1) (layer "B.Cu") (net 1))
 (segment (start 117.14 107.02) (end 117.22 107.1) (width 0.2) (layer "B.Cu") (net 1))
 (segment (start 125.6 82.88) (end 125.6 87.7) (width 1) (layer "B.Cu") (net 1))
 (segment (start 125.5 107.1) (end 125.48 107.12) (width 0.2) (layer "B.Cu") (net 1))
 (segment (start 132.3 82.86) (end 125.62 82.86) (width 1) (layer "B.Cu") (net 1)))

